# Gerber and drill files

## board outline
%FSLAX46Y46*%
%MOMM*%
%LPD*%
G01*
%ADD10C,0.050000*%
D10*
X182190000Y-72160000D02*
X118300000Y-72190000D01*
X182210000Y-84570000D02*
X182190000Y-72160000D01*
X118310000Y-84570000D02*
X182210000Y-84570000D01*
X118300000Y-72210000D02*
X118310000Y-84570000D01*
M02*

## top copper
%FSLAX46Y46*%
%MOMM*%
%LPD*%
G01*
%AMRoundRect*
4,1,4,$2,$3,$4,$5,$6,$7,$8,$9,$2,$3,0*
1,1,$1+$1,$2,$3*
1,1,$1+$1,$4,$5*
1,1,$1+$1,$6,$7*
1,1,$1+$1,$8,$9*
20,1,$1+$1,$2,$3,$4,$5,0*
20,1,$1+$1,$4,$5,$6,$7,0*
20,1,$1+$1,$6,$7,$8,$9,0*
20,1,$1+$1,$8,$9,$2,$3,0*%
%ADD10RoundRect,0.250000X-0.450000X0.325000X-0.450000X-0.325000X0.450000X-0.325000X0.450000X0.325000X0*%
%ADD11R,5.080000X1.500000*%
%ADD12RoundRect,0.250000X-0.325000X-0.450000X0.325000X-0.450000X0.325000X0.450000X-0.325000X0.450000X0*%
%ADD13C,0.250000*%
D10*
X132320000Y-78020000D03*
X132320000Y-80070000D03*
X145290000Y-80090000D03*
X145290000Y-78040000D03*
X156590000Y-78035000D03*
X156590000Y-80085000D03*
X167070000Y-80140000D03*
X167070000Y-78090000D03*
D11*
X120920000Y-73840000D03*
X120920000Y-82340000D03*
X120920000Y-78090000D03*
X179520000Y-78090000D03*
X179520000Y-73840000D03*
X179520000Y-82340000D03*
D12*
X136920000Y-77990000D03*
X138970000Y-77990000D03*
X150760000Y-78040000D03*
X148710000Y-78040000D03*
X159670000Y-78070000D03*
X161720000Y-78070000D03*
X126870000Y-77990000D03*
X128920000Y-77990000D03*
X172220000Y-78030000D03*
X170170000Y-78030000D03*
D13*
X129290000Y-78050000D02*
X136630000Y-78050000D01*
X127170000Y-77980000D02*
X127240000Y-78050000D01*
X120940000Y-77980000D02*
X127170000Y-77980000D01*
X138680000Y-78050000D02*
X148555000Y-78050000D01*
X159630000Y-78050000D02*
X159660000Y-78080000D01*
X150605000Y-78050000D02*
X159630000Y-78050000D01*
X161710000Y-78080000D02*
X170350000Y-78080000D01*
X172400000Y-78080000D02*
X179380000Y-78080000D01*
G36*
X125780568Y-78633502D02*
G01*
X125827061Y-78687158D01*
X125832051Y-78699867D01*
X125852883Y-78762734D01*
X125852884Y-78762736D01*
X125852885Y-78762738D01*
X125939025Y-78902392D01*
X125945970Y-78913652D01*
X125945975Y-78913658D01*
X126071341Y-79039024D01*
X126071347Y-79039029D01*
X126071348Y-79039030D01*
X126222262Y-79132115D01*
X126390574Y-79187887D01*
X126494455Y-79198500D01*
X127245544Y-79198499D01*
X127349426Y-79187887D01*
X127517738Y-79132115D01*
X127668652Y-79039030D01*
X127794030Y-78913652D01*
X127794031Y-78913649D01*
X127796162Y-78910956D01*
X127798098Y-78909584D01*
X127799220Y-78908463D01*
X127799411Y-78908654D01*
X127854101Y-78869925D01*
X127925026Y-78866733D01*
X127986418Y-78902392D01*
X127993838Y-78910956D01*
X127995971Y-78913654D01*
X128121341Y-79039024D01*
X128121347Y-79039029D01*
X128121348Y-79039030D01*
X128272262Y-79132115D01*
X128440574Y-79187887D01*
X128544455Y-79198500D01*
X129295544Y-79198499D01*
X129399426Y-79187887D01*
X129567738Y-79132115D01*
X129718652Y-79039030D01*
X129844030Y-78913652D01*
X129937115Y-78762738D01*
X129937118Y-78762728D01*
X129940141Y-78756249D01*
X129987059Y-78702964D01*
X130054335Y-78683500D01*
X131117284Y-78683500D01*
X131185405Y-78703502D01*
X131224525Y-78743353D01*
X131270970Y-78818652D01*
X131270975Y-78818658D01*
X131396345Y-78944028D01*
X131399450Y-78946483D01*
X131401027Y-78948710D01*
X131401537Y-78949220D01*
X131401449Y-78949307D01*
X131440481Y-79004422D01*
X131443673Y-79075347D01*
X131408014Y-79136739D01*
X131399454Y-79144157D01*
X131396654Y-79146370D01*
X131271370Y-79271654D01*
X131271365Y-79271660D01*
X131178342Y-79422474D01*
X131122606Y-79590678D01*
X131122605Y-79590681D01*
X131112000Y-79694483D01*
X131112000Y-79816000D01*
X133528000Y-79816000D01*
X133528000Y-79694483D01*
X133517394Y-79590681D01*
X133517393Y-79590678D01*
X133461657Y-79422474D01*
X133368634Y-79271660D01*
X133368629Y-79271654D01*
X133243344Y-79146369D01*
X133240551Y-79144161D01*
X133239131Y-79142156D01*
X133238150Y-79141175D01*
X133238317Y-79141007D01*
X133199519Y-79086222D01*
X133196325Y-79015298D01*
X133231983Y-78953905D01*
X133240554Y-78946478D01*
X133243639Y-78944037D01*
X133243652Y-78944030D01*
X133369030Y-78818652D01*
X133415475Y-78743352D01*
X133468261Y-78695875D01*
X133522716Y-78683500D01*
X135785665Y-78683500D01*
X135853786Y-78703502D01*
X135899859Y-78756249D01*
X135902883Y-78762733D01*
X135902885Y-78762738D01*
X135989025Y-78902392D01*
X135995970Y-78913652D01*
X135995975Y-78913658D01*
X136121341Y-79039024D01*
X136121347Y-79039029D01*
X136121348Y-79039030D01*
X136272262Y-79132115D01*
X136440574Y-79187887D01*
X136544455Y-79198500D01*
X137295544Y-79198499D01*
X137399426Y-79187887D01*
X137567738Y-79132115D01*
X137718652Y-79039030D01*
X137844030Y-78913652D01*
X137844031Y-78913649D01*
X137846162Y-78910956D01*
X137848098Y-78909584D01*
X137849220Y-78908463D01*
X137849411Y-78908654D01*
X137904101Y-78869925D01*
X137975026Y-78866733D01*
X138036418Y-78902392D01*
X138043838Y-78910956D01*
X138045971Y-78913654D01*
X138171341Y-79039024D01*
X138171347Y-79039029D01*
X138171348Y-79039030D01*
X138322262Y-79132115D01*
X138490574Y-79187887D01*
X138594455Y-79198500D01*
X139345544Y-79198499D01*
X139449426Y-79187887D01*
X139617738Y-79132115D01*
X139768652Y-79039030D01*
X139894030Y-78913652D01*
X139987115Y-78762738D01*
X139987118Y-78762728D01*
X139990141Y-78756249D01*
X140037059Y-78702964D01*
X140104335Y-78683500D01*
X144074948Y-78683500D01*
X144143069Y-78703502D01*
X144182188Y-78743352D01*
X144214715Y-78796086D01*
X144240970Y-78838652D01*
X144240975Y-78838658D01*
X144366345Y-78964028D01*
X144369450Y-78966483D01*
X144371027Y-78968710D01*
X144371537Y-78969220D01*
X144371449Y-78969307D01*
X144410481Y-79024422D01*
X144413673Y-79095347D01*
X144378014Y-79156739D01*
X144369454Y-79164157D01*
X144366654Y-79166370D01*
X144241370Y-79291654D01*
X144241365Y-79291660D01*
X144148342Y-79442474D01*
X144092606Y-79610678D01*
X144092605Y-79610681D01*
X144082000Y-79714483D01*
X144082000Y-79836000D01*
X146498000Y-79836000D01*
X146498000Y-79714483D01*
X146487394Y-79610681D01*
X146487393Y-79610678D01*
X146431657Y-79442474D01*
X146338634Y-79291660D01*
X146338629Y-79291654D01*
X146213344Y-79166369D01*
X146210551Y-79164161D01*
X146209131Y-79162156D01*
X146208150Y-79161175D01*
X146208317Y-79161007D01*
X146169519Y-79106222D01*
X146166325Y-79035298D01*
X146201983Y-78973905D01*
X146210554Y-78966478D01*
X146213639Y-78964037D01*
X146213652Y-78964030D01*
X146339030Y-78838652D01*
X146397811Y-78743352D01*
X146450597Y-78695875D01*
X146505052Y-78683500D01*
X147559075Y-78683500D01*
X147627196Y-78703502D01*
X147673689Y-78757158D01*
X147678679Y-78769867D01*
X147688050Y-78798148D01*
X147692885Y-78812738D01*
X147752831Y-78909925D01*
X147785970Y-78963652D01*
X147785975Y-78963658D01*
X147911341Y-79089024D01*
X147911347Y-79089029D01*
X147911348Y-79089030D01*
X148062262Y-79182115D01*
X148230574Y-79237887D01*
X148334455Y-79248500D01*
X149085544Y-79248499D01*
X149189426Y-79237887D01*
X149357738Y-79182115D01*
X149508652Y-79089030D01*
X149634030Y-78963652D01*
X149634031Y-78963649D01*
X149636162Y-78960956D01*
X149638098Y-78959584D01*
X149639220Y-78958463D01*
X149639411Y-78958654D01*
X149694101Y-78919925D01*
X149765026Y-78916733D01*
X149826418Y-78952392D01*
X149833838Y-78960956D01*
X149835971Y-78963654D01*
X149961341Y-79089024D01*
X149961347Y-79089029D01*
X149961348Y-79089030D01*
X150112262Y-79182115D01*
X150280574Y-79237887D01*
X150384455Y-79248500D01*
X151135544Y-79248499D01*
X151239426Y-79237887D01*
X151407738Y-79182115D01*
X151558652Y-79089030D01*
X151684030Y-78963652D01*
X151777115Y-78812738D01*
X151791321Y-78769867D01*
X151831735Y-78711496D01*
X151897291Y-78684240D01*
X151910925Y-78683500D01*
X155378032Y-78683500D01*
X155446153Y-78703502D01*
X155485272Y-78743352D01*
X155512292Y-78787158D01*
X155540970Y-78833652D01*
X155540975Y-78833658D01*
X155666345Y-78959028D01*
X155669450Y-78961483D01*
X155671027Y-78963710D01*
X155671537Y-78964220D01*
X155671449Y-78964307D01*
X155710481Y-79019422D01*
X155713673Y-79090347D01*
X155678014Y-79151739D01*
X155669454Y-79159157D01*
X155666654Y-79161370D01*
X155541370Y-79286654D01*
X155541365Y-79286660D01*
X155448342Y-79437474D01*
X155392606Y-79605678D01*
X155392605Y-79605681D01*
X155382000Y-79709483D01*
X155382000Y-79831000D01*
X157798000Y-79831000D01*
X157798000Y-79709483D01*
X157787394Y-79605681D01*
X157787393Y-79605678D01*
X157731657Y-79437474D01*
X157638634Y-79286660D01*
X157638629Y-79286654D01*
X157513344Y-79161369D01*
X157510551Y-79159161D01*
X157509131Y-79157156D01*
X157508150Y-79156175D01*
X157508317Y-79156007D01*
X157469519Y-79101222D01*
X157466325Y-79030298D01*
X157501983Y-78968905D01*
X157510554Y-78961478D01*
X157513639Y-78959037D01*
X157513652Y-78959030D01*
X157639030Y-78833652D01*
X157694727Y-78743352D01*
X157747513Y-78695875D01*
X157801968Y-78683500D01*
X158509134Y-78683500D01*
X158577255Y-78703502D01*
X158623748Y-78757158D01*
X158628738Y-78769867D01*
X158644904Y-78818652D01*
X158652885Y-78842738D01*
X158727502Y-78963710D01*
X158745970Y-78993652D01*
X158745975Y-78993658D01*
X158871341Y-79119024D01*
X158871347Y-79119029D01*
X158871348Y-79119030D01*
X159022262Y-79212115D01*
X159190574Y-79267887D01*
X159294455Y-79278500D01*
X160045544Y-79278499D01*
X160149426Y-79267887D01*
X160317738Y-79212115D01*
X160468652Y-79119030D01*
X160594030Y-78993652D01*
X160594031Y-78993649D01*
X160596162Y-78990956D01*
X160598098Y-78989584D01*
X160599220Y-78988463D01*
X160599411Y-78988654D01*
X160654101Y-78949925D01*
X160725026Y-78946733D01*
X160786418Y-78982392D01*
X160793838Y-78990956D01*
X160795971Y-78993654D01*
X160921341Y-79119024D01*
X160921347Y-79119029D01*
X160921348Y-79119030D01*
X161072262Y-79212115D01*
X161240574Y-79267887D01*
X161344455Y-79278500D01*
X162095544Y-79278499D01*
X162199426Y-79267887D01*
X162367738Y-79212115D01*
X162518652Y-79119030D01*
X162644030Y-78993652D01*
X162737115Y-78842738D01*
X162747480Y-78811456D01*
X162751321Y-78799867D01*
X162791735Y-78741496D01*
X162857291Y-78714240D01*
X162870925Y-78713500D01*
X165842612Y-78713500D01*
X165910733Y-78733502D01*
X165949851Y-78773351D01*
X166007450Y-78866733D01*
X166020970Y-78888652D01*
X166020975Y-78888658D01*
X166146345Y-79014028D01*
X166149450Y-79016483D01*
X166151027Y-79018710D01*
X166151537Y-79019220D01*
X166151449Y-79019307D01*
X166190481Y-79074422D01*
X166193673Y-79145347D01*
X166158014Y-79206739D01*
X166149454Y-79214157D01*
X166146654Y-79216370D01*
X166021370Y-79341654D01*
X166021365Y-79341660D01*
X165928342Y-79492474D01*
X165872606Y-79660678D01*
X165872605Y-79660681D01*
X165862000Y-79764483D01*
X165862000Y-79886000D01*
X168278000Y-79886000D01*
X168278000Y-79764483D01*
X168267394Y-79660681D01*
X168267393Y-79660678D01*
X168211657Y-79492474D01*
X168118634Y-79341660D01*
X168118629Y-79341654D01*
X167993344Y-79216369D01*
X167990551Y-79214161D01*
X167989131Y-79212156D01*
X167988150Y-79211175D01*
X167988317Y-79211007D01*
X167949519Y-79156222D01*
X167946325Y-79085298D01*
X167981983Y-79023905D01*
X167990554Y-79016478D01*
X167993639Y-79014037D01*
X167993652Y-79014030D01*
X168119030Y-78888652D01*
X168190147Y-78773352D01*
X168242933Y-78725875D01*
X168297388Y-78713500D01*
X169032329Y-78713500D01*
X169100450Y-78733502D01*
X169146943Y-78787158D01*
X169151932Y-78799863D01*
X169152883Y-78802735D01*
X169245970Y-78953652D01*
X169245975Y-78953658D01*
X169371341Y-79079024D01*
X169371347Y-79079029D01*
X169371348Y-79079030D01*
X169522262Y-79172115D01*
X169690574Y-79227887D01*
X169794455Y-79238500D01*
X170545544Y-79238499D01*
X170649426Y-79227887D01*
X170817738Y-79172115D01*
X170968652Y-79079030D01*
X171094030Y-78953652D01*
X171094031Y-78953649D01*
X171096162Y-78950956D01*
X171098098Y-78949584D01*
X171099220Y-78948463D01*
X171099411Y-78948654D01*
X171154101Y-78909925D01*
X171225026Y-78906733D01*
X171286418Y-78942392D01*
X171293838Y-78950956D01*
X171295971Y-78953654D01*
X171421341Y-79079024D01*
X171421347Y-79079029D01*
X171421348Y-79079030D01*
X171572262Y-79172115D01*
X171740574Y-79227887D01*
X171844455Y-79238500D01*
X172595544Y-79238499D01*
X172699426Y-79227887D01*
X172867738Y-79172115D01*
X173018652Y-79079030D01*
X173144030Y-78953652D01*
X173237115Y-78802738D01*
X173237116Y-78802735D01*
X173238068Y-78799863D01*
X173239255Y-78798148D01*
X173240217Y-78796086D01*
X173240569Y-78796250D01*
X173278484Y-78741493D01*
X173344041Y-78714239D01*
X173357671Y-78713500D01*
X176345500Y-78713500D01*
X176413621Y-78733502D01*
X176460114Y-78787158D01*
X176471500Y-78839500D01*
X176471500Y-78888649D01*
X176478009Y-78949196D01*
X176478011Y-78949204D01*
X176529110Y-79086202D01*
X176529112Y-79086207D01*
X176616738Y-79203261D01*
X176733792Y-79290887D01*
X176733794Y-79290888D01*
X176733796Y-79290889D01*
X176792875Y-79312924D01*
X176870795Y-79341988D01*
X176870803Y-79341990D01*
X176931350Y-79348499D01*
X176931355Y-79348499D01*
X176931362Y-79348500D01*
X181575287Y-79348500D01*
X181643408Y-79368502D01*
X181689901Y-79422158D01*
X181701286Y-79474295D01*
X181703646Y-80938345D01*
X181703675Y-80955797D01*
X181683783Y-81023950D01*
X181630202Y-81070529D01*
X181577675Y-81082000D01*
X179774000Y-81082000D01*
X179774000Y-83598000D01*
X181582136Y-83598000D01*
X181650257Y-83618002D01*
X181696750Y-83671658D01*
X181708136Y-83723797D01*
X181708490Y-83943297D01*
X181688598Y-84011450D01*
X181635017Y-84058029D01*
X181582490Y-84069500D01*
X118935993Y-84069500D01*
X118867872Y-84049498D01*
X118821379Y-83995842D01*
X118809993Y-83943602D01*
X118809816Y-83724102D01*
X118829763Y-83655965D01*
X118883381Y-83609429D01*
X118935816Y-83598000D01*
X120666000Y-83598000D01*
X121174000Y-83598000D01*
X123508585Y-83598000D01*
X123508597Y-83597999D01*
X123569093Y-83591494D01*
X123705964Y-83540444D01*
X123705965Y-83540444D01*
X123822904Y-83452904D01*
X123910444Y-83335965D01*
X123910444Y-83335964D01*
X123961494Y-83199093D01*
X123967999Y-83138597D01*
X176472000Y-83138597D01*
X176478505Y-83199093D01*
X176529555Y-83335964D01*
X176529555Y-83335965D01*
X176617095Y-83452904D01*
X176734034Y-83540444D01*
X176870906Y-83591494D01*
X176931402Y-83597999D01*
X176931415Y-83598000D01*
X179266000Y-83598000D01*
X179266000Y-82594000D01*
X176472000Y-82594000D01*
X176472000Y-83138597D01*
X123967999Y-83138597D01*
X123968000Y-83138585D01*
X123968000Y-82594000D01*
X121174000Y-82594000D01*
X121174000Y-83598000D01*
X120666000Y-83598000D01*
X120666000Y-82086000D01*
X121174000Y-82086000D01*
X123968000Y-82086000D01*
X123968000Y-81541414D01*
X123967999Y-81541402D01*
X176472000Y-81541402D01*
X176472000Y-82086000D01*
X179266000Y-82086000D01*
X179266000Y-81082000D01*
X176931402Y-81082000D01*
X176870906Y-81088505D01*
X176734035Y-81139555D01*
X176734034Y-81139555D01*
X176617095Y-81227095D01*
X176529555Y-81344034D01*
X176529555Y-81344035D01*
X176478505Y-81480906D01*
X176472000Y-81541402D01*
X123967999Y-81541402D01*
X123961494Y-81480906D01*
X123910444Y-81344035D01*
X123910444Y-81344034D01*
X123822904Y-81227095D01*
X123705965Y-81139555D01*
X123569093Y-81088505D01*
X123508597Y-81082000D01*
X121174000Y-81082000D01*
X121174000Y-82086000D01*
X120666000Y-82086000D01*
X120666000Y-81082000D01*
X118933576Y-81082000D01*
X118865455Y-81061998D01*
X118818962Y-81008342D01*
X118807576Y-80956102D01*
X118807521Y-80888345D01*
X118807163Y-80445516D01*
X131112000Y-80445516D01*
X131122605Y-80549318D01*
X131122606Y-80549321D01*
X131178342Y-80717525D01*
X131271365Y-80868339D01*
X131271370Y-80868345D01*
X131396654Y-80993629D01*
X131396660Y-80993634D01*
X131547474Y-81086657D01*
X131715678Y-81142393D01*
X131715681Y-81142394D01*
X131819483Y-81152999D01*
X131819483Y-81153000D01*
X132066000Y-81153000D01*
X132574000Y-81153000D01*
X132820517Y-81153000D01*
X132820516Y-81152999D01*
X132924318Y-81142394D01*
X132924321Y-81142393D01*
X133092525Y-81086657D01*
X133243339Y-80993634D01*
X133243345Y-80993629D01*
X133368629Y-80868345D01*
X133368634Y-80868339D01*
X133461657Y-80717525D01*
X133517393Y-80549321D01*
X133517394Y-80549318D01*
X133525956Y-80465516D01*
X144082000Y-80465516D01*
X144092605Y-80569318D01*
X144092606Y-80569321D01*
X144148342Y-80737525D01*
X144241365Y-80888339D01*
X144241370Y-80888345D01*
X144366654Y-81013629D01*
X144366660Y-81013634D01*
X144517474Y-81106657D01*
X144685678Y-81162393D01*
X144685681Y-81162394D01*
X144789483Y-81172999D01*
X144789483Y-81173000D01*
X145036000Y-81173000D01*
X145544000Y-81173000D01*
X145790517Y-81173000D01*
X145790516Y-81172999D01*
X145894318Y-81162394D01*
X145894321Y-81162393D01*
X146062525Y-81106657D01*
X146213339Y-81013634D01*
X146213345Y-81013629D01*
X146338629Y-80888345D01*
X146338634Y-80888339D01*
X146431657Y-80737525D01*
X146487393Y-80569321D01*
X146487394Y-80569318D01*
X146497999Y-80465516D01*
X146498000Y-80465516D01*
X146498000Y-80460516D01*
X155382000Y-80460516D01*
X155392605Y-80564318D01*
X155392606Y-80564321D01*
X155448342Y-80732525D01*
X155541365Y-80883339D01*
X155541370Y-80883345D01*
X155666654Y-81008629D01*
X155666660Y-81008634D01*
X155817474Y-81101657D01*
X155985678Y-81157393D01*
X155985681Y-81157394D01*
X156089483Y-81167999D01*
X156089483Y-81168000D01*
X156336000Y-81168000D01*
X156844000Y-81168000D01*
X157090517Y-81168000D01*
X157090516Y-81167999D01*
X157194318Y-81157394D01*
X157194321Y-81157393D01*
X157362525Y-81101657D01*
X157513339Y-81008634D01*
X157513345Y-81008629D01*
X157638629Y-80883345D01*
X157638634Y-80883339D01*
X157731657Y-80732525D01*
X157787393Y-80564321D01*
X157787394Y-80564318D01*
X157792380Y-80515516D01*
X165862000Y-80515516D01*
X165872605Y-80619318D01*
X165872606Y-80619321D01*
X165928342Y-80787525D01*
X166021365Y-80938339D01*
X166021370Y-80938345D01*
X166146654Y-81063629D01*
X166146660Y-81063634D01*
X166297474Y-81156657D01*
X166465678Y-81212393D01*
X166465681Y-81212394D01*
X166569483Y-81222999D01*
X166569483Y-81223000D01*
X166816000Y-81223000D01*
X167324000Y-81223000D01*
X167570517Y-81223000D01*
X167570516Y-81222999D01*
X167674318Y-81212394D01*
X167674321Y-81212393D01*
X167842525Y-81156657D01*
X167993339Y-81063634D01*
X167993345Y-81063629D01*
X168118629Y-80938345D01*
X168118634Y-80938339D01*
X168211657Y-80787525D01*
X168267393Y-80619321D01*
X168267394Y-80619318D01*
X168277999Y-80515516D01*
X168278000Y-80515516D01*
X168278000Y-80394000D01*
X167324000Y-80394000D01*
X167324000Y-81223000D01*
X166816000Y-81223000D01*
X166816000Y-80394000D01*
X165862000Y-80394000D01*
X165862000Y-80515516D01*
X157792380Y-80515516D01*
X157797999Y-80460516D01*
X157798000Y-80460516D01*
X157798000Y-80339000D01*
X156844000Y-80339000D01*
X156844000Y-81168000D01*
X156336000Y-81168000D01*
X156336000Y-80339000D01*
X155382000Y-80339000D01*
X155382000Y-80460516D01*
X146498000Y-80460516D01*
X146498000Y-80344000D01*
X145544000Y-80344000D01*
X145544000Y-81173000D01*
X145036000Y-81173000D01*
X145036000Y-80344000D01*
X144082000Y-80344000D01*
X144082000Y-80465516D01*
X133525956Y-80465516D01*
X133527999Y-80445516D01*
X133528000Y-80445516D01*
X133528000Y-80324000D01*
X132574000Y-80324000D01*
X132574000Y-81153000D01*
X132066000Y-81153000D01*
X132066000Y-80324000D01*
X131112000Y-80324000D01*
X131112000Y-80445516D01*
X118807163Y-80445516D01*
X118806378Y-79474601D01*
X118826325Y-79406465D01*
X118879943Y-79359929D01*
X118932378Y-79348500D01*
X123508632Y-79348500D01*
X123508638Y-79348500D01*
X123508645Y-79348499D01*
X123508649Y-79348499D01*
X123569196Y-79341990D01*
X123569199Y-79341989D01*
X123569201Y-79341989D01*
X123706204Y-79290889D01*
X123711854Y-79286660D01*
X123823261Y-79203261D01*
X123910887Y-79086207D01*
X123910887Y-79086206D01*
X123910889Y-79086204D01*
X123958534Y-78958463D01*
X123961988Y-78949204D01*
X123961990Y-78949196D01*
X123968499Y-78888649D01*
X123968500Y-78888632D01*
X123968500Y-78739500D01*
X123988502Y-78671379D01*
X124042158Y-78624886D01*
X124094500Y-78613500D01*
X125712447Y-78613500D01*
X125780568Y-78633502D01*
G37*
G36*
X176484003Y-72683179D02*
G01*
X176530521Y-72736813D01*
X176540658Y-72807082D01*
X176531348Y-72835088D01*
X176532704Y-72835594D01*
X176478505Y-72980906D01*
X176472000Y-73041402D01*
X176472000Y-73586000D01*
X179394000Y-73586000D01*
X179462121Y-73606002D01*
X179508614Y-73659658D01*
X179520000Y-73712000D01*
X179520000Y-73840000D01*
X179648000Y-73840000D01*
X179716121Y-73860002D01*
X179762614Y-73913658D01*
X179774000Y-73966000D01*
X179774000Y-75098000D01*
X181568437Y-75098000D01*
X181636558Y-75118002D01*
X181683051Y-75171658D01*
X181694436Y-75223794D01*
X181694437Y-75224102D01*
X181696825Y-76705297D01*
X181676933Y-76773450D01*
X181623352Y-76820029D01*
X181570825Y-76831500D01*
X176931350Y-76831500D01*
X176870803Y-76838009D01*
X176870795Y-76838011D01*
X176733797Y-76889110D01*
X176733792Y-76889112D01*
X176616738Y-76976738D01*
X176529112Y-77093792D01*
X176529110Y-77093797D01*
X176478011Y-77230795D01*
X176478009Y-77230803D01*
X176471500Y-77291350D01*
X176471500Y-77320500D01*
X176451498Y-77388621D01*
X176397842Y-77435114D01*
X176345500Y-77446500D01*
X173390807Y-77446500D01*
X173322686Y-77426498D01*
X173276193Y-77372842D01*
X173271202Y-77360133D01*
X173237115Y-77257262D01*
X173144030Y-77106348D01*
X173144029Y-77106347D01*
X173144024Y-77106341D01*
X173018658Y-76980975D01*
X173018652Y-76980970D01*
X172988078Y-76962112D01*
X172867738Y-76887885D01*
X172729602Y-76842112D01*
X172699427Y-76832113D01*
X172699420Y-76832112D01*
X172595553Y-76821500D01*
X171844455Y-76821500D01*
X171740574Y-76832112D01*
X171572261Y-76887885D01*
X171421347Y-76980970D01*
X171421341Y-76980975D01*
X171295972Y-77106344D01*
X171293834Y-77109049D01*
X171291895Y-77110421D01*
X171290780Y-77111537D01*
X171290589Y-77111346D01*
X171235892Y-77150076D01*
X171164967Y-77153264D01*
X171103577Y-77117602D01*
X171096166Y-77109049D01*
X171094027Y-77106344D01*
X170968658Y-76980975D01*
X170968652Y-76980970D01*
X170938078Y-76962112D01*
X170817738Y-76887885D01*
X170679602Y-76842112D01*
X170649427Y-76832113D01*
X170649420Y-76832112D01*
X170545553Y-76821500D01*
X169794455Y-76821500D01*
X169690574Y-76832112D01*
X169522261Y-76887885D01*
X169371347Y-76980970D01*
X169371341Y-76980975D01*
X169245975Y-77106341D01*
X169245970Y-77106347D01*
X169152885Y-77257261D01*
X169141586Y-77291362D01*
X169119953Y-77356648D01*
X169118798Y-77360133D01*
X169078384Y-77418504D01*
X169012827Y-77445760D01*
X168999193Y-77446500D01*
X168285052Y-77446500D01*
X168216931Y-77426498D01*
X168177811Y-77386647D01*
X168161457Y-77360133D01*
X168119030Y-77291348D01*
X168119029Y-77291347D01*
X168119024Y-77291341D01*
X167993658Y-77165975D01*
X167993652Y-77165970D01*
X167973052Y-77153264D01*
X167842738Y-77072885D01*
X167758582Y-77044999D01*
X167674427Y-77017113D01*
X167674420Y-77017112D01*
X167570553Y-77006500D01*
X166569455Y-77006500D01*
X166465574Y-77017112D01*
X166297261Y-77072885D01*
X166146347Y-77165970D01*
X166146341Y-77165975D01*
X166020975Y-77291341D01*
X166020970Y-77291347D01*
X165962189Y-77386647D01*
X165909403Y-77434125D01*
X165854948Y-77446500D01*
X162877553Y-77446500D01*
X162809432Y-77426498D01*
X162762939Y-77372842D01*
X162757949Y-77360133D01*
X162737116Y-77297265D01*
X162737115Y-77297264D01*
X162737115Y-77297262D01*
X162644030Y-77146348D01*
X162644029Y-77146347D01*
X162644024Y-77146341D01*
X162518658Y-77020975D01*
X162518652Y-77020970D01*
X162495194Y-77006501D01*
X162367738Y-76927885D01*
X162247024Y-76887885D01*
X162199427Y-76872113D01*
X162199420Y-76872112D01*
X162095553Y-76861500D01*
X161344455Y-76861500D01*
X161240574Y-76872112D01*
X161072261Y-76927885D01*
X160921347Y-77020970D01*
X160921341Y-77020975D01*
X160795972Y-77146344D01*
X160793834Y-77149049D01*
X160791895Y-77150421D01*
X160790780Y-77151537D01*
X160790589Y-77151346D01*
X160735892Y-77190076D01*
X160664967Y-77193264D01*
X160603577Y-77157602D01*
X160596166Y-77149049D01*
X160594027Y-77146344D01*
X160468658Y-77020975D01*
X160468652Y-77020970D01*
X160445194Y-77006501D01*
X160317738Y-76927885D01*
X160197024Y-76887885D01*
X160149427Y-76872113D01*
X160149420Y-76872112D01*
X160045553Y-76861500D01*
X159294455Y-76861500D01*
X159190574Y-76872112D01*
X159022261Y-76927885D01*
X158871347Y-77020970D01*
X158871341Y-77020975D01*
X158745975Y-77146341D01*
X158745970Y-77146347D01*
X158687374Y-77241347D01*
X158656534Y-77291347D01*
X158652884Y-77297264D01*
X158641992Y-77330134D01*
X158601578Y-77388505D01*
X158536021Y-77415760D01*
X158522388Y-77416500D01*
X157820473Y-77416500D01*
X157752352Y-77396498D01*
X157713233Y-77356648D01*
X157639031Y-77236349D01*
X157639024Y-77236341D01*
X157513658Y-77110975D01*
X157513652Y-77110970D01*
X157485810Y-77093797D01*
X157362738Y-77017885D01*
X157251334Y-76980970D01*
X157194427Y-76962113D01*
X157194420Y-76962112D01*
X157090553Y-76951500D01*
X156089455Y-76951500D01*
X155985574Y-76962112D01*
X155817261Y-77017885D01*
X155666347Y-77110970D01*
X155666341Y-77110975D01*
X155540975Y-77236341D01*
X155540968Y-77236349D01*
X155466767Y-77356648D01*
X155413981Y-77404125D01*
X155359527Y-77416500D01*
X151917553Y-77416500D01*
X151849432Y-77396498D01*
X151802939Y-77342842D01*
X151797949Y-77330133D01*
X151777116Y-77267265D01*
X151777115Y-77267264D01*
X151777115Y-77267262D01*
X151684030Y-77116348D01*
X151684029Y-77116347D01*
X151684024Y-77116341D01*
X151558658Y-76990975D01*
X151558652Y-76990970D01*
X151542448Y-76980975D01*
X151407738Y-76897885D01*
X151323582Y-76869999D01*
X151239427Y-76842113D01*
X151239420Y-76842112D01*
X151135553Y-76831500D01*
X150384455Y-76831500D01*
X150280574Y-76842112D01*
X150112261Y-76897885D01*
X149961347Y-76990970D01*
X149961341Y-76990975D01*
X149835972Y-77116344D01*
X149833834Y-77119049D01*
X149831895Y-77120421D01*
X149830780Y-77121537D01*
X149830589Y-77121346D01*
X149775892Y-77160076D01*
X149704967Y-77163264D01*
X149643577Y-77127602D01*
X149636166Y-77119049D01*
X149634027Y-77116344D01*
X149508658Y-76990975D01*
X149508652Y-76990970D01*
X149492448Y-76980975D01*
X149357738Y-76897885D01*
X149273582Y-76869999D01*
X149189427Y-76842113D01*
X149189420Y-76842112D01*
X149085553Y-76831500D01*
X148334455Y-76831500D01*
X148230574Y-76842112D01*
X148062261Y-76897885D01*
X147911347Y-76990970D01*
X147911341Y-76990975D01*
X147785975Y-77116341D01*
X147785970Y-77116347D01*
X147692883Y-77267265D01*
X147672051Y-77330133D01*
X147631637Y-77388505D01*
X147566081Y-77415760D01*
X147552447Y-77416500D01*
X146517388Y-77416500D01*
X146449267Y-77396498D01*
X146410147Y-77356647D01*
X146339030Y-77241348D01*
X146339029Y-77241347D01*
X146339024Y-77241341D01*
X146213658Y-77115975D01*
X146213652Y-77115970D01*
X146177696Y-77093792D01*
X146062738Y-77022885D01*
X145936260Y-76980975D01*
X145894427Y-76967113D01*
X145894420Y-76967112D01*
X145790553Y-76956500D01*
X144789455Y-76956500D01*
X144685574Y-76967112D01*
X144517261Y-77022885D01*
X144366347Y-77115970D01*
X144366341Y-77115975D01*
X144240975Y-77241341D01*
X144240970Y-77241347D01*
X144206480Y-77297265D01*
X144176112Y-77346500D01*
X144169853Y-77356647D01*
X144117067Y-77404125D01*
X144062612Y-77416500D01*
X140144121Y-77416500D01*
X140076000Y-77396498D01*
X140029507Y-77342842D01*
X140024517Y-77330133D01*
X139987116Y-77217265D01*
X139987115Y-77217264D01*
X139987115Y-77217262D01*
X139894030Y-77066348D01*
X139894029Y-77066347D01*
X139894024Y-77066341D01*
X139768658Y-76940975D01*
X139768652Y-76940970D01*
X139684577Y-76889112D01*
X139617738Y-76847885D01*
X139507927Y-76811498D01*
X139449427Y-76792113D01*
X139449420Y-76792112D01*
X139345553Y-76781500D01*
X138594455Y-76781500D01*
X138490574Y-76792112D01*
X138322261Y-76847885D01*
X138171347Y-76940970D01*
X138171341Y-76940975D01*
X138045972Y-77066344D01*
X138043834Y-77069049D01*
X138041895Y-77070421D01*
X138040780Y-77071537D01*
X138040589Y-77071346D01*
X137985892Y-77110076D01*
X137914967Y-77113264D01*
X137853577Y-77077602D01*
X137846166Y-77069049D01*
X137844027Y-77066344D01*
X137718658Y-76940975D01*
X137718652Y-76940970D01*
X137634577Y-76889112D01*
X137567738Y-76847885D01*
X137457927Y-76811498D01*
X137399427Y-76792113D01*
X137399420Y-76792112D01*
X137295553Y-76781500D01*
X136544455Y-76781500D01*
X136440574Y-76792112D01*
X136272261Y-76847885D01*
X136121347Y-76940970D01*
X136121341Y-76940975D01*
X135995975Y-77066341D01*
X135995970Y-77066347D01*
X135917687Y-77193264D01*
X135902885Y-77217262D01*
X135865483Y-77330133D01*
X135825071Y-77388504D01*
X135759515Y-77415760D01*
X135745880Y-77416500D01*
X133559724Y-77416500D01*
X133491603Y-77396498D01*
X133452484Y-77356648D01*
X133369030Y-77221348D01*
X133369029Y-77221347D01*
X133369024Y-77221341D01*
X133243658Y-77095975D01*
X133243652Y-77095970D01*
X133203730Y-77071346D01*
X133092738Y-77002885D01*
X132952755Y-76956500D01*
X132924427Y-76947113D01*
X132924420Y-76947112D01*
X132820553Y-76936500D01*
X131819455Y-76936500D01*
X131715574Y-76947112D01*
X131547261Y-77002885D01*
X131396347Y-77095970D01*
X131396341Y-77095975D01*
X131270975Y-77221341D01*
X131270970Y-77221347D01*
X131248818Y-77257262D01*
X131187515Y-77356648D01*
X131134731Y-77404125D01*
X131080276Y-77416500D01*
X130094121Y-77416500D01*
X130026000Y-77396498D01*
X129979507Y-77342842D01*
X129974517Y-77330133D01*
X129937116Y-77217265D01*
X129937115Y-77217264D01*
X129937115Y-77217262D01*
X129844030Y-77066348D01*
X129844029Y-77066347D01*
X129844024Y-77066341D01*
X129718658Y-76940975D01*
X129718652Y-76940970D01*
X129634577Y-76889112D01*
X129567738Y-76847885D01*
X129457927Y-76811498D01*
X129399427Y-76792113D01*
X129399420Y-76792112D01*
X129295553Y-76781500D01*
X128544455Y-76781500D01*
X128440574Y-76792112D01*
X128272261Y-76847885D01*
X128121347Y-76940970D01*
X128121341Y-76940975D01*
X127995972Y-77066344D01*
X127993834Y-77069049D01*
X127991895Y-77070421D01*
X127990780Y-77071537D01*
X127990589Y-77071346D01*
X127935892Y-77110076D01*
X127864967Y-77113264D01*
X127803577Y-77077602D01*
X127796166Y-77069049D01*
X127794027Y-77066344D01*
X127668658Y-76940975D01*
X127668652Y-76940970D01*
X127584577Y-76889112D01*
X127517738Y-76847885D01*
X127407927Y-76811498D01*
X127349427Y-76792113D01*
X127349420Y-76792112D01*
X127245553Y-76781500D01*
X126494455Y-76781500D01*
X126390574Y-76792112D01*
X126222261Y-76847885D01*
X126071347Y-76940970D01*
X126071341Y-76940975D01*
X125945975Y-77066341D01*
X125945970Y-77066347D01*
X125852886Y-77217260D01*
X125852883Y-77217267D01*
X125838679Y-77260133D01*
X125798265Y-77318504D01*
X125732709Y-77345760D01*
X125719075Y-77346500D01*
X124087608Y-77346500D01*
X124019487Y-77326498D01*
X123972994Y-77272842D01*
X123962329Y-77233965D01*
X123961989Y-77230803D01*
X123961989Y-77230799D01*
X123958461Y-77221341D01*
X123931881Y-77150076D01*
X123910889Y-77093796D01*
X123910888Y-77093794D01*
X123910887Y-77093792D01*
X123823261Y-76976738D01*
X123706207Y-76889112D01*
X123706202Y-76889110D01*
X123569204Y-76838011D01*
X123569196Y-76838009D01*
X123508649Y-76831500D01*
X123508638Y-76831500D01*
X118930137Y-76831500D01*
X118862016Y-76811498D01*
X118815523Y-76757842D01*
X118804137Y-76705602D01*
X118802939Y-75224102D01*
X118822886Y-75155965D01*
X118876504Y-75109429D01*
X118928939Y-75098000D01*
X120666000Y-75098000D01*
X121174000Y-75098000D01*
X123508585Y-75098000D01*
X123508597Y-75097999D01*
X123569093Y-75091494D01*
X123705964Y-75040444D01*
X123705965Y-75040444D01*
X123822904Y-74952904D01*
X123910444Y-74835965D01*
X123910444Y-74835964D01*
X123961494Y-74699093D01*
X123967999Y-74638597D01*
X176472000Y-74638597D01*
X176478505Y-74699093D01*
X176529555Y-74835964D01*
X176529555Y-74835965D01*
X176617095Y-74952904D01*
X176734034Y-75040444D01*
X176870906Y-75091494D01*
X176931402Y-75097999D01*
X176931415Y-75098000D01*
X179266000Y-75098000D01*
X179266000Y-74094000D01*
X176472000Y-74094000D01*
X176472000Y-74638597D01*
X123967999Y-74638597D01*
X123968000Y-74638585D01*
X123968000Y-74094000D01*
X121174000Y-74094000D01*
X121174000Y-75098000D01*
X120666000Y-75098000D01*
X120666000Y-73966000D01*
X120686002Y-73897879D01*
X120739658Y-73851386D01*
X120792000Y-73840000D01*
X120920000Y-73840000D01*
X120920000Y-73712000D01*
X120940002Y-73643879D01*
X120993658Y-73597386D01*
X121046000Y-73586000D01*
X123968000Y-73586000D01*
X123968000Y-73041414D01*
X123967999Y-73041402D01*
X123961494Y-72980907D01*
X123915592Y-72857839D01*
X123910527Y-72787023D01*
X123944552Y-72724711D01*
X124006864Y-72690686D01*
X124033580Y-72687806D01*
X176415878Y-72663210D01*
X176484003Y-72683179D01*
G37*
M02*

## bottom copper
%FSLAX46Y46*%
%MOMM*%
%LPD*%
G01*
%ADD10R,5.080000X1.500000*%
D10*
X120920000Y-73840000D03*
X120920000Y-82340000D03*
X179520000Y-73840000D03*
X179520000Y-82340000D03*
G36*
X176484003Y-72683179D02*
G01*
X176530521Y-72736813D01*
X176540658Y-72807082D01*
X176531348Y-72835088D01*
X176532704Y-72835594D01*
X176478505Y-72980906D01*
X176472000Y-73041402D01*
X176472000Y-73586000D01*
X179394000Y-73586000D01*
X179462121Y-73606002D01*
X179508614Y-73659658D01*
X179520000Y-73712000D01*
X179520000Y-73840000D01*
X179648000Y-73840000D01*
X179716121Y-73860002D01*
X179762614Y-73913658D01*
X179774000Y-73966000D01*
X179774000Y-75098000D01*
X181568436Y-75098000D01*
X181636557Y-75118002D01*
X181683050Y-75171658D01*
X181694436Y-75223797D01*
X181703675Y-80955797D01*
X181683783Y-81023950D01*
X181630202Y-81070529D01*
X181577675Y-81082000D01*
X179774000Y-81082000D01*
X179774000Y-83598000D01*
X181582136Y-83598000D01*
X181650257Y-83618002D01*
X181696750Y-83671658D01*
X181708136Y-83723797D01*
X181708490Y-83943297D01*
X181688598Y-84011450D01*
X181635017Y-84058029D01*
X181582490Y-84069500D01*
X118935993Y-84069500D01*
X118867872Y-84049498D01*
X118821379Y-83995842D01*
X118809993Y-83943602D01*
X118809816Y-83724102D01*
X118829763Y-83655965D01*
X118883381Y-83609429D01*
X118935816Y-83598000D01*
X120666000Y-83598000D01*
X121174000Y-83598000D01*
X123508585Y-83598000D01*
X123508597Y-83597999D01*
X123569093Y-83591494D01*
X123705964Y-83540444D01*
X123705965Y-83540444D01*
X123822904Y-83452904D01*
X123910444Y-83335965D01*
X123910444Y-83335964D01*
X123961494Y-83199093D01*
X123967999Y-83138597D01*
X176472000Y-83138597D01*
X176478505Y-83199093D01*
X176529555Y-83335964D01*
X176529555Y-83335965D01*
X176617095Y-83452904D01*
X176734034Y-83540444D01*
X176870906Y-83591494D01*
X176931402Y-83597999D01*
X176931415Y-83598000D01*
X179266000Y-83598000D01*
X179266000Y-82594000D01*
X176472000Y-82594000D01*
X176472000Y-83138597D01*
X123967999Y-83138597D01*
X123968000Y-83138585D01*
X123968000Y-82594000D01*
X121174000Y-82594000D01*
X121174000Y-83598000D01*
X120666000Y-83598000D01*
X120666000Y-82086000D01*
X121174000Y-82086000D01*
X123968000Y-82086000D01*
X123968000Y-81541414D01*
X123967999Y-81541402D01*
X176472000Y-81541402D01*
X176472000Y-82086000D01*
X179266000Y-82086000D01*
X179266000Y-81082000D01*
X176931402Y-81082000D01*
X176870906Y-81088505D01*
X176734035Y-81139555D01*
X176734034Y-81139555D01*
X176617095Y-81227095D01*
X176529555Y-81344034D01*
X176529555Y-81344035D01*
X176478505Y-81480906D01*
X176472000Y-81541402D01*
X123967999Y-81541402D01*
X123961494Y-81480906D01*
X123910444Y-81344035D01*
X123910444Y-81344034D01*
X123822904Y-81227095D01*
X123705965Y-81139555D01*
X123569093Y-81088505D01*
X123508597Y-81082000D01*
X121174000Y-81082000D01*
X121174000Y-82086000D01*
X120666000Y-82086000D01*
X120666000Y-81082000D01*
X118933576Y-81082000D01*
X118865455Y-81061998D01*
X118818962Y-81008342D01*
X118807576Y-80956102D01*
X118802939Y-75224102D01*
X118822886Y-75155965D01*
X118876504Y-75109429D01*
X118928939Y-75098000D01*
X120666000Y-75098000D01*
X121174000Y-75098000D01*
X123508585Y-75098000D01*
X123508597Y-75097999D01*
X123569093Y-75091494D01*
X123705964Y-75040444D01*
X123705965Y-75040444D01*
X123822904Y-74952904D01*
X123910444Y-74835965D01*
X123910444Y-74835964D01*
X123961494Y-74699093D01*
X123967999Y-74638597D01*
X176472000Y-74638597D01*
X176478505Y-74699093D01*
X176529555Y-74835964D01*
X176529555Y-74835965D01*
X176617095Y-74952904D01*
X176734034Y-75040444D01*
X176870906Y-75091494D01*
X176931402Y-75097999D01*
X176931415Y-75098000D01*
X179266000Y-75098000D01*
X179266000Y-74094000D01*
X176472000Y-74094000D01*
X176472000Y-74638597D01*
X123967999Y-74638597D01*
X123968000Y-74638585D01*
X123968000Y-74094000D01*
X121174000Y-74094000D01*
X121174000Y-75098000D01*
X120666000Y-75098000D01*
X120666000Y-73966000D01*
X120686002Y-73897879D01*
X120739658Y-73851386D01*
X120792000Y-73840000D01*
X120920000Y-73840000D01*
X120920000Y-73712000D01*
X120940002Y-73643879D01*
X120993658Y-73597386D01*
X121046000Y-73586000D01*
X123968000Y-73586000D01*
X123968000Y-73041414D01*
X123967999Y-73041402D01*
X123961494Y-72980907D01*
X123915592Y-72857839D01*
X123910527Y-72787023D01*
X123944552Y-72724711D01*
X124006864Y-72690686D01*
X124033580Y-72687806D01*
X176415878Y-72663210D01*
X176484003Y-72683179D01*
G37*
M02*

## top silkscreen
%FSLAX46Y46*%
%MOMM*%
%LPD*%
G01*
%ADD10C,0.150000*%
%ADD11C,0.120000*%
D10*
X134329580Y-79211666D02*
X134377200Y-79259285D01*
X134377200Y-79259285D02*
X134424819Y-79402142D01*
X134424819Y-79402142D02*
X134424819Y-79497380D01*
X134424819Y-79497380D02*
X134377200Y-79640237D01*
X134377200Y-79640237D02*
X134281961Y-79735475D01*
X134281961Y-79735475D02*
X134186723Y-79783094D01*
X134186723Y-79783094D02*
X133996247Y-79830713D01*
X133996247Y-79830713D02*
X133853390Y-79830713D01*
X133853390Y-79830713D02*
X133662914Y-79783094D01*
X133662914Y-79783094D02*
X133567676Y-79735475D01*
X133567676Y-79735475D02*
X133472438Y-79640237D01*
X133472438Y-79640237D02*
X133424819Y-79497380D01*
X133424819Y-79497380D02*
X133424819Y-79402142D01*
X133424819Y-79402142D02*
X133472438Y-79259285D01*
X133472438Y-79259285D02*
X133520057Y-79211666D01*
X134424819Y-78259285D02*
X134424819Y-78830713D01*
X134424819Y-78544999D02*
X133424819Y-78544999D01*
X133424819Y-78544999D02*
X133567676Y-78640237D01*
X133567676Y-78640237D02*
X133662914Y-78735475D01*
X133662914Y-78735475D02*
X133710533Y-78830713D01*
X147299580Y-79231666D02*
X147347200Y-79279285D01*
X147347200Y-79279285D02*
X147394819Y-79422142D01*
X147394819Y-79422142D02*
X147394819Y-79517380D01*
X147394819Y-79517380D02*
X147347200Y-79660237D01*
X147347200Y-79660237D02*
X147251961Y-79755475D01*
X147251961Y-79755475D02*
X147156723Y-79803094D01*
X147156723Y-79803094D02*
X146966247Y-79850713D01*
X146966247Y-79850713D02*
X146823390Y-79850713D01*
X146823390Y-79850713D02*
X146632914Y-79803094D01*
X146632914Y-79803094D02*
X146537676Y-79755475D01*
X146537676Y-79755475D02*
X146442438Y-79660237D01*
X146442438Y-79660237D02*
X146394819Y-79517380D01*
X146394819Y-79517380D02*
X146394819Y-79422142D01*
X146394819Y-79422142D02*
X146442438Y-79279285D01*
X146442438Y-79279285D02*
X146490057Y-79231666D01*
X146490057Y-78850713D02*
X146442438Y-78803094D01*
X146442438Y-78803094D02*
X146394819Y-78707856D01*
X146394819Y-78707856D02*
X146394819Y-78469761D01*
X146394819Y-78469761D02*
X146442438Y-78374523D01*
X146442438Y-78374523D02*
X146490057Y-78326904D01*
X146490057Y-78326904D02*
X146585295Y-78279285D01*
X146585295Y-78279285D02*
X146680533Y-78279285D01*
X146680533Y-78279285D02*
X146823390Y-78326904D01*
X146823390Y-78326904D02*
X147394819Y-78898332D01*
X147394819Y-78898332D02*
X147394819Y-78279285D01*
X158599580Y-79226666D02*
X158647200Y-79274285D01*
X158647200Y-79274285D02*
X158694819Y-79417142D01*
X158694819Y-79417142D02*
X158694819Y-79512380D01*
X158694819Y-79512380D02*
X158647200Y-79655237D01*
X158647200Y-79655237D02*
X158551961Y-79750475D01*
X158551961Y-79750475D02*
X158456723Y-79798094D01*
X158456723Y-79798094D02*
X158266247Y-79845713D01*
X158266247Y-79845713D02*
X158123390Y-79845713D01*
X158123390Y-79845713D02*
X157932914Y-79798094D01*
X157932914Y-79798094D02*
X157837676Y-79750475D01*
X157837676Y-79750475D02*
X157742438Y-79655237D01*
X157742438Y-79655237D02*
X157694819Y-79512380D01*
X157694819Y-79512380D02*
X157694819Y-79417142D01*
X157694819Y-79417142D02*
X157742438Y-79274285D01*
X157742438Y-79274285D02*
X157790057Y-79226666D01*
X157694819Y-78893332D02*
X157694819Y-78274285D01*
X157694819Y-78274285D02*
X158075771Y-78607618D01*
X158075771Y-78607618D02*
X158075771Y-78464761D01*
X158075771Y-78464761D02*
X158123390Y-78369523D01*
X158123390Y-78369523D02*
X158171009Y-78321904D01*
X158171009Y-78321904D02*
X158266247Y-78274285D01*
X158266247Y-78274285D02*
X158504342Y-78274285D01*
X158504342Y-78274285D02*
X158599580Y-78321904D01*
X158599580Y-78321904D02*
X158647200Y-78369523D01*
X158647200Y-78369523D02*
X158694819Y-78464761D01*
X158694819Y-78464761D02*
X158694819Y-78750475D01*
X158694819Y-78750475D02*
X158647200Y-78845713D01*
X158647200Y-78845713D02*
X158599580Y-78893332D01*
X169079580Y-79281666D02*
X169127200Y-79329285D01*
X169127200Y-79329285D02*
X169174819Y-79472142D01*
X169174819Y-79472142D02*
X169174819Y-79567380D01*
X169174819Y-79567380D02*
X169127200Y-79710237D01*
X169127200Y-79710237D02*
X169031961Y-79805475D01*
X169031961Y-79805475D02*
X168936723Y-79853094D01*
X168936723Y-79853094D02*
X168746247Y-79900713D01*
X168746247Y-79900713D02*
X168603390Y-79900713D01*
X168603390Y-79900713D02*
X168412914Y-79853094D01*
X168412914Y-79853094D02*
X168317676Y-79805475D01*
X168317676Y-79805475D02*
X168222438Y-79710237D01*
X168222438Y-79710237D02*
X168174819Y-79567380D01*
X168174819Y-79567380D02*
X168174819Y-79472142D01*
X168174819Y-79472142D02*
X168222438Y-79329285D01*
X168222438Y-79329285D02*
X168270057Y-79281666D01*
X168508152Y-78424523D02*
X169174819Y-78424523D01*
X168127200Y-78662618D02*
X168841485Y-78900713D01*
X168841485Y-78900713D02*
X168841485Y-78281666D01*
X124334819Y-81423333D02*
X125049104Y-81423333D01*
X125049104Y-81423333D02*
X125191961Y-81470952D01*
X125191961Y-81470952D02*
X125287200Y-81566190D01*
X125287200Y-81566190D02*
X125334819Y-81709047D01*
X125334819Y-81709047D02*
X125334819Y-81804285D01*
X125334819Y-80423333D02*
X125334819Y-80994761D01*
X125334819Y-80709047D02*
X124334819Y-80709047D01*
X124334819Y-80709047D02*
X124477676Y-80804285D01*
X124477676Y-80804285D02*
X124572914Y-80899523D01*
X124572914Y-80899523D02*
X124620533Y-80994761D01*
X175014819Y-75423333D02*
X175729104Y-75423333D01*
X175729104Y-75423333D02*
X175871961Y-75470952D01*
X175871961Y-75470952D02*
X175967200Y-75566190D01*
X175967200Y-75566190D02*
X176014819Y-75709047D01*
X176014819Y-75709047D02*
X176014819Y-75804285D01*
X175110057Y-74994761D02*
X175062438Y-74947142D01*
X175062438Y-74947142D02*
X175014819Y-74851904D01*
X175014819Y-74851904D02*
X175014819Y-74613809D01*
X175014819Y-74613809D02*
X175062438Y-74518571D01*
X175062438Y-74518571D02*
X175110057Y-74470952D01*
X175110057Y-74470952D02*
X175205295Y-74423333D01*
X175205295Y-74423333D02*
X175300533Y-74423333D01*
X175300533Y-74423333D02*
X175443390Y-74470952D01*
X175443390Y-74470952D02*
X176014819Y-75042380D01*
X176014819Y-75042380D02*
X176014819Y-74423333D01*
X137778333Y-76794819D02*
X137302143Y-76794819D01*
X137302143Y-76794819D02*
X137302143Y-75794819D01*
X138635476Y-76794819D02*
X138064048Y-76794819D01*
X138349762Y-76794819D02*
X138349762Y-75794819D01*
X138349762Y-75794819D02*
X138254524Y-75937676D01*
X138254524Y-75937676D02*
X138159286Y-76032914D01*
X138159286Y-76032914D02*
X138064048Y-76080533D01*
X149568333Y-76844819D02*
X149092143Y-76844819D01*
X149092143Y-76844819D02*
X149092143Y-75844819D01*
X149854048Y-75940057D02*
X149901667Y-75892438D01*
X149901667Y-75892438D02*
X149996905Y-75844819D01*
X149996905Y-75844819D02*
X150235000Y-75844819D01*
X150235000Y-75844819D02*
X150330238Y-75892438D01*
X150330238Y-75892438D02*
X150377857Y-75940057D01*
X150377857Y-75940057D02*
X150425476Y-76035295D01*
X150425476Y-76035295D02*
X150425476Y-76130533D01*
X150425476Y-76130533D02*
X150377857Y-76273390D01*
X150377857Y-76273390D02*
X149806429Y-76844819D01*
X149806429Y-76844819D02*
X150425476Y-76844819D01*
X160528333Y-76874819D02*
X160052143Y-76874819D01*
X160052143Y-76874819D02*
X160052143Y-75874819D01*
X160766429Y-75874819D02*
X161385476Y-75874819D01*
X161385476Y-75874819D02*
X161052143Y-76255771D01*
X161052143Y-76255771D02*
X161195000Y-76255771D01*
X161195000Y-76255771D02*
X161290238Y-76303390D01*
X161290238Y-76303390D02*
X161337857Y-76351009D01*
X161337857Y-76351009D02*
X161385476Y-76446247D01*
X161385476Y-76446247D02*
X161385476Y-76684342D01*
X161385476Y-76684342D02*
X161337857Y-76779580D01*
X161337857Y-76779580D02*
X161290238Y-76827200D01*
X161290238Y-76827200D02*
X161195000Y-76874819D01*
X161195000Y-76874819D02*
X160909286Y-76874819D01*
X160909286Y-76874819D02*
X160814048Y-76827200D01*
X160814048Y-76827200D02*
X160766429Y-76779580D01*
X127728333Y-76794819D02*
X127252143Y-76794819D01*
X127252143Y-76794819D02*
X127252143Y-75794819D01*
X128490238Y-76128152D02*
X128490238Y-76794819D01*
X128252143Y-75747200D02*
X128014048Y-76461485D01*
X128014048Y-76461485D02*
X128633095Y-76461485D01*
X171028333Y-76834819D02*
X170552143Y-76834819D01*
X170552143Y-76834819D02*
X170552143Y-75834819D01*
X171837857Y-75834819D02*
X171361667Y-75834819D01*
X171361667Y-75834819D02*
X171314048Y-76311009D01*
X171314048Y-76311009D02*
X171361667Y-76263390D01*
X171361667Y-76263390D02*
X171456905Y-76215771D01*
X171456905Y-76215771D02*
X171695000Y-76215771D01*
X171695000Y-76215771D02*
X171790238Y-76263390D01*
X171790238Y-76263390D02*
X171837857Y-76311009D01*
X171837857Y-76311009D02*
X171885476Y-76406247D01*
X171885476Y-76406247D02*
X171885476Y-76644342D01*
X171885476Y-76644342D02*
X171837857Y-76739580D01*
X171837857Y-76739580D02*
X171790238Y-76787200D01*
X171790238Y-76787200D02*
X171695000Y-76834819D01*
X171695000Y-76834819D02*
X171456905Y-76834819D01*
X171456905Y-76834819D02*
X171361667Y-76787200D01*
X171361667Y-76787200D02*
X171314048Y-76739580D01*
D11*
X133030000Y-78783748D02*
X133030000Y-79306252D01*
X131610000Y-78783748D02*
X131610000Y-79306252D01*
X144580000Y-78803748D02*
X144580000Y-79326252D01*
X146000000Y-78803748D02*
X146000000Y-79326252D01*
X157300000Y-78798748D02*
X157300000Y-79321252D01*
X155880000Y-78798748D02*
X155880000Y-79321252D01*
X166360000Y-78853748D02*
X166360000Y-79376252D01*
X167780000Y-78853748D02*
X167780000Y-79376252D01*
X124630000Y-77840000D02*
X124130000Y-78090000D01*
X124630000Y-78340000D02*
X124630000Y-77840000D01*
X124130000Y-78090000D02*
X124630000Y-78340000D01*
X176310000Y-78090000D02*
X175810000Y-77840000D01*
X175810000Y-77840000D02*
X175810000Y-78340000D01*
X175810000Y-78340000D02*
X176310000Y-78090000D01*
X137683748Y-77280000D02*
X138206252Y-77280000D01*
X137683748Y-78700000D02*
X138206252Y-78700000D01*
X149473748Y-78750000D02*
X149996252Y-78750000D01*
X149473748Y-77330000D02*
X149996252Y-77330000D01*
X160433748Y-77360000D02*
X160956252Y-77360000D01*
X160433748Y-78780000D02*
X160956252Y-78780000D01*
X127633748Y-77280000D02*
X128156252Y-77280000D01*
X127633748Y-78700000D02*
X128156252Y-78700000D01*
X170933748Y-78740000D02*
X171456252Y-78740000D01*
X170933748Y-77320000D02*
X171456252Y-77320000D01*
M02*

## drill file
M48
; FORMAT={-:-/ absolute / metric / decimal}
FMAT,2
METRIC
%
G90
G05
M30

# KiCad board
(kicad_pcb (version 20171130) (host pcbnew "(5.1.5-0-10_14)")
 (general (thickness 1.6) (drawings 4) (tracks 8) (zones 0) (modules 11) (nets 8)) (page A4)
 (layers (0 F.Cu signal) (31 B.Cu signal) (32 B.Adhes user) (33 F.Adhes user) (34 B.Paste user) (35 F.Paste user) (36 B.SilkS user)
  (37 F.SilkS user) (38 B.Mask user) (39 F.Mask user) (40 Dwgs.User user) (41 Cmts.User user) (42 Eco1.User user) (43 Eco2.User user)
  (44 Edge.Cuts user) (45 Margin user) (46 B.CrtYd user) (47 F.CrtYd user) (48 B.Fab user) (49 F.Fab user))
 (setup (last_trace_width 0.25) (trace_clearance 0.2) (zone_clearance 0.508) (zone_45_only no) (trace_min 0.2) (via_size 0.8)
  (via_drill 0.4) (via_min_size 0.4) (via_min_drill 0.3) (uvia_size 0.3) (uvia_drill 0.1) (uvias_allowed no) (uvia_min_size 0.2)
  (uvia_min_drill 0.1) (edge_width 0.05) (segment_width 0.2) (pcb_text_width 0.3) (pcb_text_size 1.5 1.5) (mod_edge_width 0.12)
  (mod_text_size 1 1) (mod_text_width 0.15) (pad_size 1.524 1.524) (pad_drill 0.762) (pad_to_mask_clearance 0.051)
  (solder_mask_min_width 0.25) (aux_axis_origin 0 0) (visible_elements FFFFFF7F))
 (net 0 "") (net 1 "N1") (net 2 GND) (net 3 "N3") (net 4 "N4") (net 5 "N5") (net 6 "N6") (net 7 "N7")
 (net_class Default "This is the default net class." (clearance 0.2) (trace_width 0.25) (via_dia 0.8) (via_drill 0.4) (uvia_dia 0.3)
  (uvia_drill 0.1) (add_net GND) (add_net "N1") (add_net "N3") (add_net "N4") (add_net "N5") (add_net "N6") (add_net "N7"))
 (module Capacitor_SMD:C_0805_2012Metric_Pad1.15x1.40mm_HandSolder (layer F.Cu) (at 132.32 79.045 270)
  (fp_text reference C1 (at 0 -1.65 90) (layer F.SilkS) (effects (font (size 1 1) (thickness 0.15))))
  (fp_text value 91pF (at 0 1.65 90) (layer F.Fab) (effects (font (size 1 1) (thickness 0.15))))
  (fp_line (start -0.261252 -0.71) (end 0.261252 -0.71) (layer F.SilkS) (width 0.12))
  (fp_line (start -0.261252 0.71) (end 0.261252 0.71) (layer F.SilkS) (width 0.12))
  (pad 1 smd roundrect (at -1.025 0 270) (size 1.15 1.4) (layers F.Cu F.Paste F.Mask) (roundrect_rratio 0.217391) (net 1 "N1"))
  (pad 2 smd roundrect (at 1.025 0 270) (size 1.15 1.4) (layers F.Cu F.Paste F.Mask) (roundrect_rratio 0.217391) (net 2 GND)))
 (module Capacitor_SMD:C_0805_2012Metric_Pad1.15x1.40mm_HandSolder (layer F.Cu) (at 145.29 79.065 270)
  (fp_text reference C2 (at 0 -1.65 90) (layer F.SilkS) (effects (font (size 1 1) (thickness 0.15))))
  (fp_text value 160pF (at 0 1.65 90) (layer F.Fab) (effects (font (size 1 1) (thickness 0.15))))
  (fp_line (start -0.261252 0.71) (end 0.261252 0.71) (layer F.SilkS) (width 0.12))
  (fp_line (start -0.261252 -0.71) (end 0.261252 -0.71) (layer F.SilkS) (width 0.12))
  (pad 2 smd roundrect (at 1.025 0 270) (size 1.15 1.4) (layers F.Cu F.Paste F.Mask) (roundrect_rratio 0.217391) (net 2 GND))
  (pad 1 smd roundrect (at -1.025 0 270) (size 1.15 1.4) (layers F.Cu F.Paste F.Mask) (roundrect_rratio 0.217391) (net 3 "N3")))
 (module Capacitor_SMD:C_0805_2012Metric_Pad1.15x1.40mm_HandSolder (layer F.Cu) (at 156.59 79.06 270)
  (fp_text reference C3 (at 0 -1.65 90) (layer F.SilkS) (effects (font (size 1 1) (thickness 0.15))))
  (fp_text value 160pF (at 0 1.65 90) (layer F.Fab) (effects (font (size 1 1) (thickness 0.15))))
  (fp_line (start -0.261252 -0.71) (end 0.261252 -0.71) (layer F.SilkS) (width 0.12))
  (fp_line (start -0.261252 0.71) (end 0.261252 0.71) (layer F.SilkS) (width 0.12))
  (pad 1 smd roundrect (at -1.025 0 270) (size 1.15 1.4) (layers F.Cu F.Paste F.Mask) (roundrect_rratio 0.217391) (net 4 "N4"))
  (pad 2 smd roundrect (at 1.025 0 270) (size 1.15 1.4) (layers F.Cu F.Paste F.Mask) (roundrect_rratio 0.217391) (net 2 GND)))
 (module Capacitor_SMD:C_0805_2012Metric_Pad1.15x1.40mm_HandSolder (layer F.Cu) (at 167.07 79.115 270)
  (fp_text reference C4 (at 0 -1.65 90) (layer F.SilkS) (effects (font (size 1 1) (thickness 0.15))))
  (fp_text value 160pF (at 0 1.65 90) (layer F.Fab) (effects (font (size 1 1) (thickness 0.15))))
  (fp_line (start -0.261252 0.71) (end 0.261252 0.71) (layer F.SilkS) (width 0.12))
  (fp_line (start -0.261252 -0.71) (end 0.261252 -0.71) (layer F.SilkS) (width 0.12))
  (pad 2 smd roundrect (at 1.025 0 270) (size 1.15 1.4) (layers F.Cu F.Paste F.Mask) (roundrect_rratio 0.217391) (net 2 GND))
  (pad 1 smd roundrect (at -1.025 0 270) (size 1.15 1.4) (layers F.Cu F.Paste F.Mask) (roundrect_rratio 0.217391) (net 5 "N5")))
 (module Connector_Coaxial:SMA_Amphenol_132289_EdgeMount (layer F.Cu) (at 120.92 78.09 180)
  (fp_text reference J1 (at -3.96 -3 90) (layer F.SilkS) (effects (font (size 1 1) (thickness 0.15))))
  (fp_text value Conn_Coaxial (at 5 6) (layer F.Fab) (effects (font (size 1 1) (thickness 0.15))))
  (fp_line (start -3.71 0.25) (end -3.21 0) (layer F.SilkS) (width 0.12))
  (fp_line (start -3.71 -0.25) (end -3.71 0.25) (layer F.SilkS) (width 0.12))
  (fp_line (start -3.21 0) (end -3.71 -0.25) (layer F.SilkS) (width 0.12))
  (pad 2 smd rect (at 0 4.25 270) (size 1.5 5.08) (layers B.Cu B.Paste B.Mask) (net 2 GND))
  (pad 2 smd rect (at 0 -4.25 270) (size 1.5 5.08) (layers B.Cu B.Paste B.Mask) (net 2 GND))
  (pad 2 smd rect (at 0 4.25 270) (size 1.5 5.08) (layers F.Cu F.Paste F.Mask) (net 2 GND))
  (pad 2 smd rect (at 0 -4.25 270) (size 1.5 5.08) (layers F.Cu F.Paste F.Mask) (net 2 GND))
  (pad 1 smd rect (at 0 0 270) (size 1.5 5.08) (layers F.Cu F.Paste F.Mask) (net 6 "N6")))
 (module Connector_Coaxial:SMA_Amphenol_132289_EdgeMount (layer F.Cu) (at 179.52 78.09)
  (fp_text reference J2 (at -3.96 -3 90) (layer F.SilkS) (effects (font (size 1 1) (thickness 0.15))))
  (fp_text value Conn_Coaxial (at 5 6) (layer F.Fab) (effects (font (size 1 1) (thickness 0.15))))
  (fp_line (start -3.21 0) (end -3.71 -0.25) (layer F.SilkS) (width 0.12))
  (fp_line (start -3.71 -0.25) (end -3.71 0.25) (layer F.SilkS) (width 0.12))
  (fp_line (start -3.71 0.25) (end -3.21 0) (layer F.SilkS) (width 0.12))
  (pad 1 smd rect (at 0 0 90) (size 1.5 5.08) (layers F.Cu F.Paste F.Mask) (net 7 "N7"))
  (pad 2 smd rect (at 0 -4.25 90) (size 1.5 5.08) (layers F.Cu F.Paste F.Mask) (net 2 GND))
  (pad 2 smd rect (at 0 4.25 90) (size 1.5 5.08) (layers F.Cu F.Paste F.Mask) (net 2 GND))
  (pad 2 smd rect (at 0 -4.25 90) (size 1.5 5.08) (layers B.Cu B.Paste B.Mask) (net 2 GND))
  (pad 2 smd rect (at 0 4.25 90) (size 1.5 5.08) (layers B.Cu B.Paste B.Mask) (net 2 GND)))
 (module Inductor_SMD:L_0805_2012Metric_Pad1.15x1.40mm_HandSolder (layer F.Cu) (at 137.945 77.99)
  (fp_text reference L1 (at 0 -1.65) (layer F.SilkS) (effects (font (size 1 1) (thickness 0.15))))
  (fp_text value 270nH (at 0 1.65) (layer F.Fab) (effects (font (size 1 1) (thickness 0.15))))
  (fp_line (start -0.261252 -0.71) (end 0.261252 -0.71) (layer F.SilkS) (width 0.12))
  (fp_line (start -0.261252 0.71) (end 0.261252 0.71) (layer F.SilkS) (width 0.12))
  (pad 1 smd roundrect (at -1.025 0) (size 1.15 1.4) (layers F.Cu F.Paste F.Mask) (roundrect_rratio 0.217391) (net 1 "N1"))
  (pad 2 smd roundrect (at 1.025 0) (size 1.15 1.4) (layers F.Cu F.Paste F.Mask) (roundrect_rratio 0.217391) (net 3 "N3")))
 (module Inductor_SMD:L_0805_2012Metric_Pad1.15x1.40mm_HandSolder (layer F.Cu) (at 149.735 78.04)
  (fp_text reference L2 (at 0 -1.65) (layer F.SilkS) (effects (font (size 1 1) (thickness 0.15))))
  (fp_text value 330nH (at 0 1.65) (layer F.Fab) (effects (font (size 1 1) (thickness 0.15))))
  (fp_line (start -0.261252 0.71) (end 0.261252 0.71) (layer F.SilkS) (width 0.12))
  (fp_line (start -0.261252 -0.71) (end 0.261252 -0.71) (layer F.SilkS) (width 0.12))
  (pad 2 smd roundrect (at 1.025 0) (size 1.15 1.4) (layers F.Cu F.Paste F.Mask) (roundrect_rratio 0.217391) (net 4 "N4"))
  (pad 1 smd roundrect (at -1.025 0) (size 1.15 1.4) (layers F.Cu F.Paste F.Mask) (roundrect_rratio 0.217391) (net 3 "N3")))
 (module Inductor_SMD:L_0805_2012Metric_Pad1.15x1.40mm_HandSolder (layer F.Cu) (at 160.695 78.07)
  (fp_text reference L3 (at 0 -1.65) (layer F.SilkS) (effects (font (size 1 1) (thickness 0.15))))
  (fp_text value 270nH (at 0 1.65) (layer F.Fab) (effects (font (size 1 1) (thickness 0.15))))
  (fp_line (start -0.261252 -0.71) (end 0.261252 -0.71) (layer F.SilkS) (width 0.12))
  (fp_line (start -0.261252 0.71) (end 0.261252 0.71) (layer F.SilkS) (width 0.12))
  (pad 1 smd roundrect (at -1.025 0) (size 1.15 1.4) (layers F.Cu F.Paste F.Mask) (roundrect_rratio 0.217391) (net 4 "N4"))
  (pad 2 smd roundrect (at 1.025 0) (size 1.15 1.4) (layers F.Cu F.Paste F.Mask) (roundrect_rratio 0.217391) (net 5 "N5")))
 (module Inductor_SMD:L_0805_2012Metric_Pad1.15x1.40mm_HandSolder (layer F.Cu) (at 127.895 77.99)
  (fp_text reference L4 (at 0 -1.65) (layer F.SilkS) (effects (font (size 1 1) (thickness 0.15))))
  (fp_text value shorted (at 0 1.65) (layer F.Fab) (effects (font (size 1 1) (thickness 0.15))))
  (fp_line (start -0.261252 -0.71) (end 0.261252 -0.71) (layer F.SilkS) (width 0.12))
  (fp_line (start -0.261252 0.71) (end 0.261252 0.71) (layer F.SilkS) (width 0.12))
  (pad 1 smd roundrect (at -1.025 0) (size 1.15 1.4) (layers F.Cu F.Paste F.Mask) (roundrect_rratio 0.217391) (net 6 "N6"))
  (pad 2 smd roundrect (at 1.025 0) (size 1.15 1.4) (layers F.Cu F.Paste F.Mask) (roundrect_rratio 0.217391) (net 1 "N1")))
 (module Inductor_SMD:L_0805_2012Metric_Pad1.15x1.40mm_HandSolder (layer F.Cu) (at 171.195 78.03)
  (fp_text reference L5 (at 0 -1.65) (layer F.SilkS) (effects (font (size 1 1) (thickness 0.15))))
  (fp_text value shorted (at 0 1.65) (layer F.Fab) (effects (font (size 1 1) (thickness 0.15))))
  (fp_line (start -0.261252 0.71) (end 0.261252 0.71) (layer F.SilkS) (width 0.12))
  (fp_line (start -0.261252 -0.71) (end 0.261252 -0.71) (layer F.SilkS) (width 0.12))
  (pad 2 smd roundrect (at 1.025 0) (size 1.15 1.4) (layers F.Cu F.Paste F.Mask) (roundrect_rratio 0.217391) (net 7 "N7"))
  (pad 1 smd roundrect (at -1.025 0) (size 1.15 1.4) (layers F.Cu F.Paste F.Mask) (roundrect_rratio 0.217391) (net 5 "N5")))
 (gr_line (start 182.19 72.16) (end 118.3 72.19) (layer Edge.Cuts) (width 0.05))
 (gr_line (start 182.21 84.57) (end 182.19 72.16) (layer Edge.Cuts) (width 0.05))
 (gr_line (start 118.31 84.57) (end 182.21 84.57) (layer Edge.Cuts) (width 0.05))
 (gr_line (start 118.3 72.21) (end 118.31 84.57) (layer Edge.Cuts) (width 0.05))
 (segment (start 129.29 78.05) (end 136.63 78.05) (width 0.25) (layer F.Cu) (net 1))
 (segment (start 127.17 77.98) (end 127.24 78.05) (width 0.25) (layer F.Cu) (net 6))
 (segment (start 120.94 77.98) (end 127.17 77.98) (width 0.25) (layer F.Cu) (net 6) (status 10))
 (segment (start 138.68 78.05) (end 148.555 78.05) (width 0.25) (layer F.Cu) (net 3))
 (segment (start 159.63 78.05) (end 159.66 78.08) (width 0.25) (layer F.Cu) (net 4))
 (segment (start 150.605 78.05) (end 159.63 78.05) (width 0.25) (layer F.Cu) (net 4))
 (segment (start 161.71 78.08) (end 170.35 78.08) (width 0.25) (layer F.Cu) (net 5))
 (segment (start 172.4 78.08) (end 179.38 78.08) (width 0.25) (layer F.Cu) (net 7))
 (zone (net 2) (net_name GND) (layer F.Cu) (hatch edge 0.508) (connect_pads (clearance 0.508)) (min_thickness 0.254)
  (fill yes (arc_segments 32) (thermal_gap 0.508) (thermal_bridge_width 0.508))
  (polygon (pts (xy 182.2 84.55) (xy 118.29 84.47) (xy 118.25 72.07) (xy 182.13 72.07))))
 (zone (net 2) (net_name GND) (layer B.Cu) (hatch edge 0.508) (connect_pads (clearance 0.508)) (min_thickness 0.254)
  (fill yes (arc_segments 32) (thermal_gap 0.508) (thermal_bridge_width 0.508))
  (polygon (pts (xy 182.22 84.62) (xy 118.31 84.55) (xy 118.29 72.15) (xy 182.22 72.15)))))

